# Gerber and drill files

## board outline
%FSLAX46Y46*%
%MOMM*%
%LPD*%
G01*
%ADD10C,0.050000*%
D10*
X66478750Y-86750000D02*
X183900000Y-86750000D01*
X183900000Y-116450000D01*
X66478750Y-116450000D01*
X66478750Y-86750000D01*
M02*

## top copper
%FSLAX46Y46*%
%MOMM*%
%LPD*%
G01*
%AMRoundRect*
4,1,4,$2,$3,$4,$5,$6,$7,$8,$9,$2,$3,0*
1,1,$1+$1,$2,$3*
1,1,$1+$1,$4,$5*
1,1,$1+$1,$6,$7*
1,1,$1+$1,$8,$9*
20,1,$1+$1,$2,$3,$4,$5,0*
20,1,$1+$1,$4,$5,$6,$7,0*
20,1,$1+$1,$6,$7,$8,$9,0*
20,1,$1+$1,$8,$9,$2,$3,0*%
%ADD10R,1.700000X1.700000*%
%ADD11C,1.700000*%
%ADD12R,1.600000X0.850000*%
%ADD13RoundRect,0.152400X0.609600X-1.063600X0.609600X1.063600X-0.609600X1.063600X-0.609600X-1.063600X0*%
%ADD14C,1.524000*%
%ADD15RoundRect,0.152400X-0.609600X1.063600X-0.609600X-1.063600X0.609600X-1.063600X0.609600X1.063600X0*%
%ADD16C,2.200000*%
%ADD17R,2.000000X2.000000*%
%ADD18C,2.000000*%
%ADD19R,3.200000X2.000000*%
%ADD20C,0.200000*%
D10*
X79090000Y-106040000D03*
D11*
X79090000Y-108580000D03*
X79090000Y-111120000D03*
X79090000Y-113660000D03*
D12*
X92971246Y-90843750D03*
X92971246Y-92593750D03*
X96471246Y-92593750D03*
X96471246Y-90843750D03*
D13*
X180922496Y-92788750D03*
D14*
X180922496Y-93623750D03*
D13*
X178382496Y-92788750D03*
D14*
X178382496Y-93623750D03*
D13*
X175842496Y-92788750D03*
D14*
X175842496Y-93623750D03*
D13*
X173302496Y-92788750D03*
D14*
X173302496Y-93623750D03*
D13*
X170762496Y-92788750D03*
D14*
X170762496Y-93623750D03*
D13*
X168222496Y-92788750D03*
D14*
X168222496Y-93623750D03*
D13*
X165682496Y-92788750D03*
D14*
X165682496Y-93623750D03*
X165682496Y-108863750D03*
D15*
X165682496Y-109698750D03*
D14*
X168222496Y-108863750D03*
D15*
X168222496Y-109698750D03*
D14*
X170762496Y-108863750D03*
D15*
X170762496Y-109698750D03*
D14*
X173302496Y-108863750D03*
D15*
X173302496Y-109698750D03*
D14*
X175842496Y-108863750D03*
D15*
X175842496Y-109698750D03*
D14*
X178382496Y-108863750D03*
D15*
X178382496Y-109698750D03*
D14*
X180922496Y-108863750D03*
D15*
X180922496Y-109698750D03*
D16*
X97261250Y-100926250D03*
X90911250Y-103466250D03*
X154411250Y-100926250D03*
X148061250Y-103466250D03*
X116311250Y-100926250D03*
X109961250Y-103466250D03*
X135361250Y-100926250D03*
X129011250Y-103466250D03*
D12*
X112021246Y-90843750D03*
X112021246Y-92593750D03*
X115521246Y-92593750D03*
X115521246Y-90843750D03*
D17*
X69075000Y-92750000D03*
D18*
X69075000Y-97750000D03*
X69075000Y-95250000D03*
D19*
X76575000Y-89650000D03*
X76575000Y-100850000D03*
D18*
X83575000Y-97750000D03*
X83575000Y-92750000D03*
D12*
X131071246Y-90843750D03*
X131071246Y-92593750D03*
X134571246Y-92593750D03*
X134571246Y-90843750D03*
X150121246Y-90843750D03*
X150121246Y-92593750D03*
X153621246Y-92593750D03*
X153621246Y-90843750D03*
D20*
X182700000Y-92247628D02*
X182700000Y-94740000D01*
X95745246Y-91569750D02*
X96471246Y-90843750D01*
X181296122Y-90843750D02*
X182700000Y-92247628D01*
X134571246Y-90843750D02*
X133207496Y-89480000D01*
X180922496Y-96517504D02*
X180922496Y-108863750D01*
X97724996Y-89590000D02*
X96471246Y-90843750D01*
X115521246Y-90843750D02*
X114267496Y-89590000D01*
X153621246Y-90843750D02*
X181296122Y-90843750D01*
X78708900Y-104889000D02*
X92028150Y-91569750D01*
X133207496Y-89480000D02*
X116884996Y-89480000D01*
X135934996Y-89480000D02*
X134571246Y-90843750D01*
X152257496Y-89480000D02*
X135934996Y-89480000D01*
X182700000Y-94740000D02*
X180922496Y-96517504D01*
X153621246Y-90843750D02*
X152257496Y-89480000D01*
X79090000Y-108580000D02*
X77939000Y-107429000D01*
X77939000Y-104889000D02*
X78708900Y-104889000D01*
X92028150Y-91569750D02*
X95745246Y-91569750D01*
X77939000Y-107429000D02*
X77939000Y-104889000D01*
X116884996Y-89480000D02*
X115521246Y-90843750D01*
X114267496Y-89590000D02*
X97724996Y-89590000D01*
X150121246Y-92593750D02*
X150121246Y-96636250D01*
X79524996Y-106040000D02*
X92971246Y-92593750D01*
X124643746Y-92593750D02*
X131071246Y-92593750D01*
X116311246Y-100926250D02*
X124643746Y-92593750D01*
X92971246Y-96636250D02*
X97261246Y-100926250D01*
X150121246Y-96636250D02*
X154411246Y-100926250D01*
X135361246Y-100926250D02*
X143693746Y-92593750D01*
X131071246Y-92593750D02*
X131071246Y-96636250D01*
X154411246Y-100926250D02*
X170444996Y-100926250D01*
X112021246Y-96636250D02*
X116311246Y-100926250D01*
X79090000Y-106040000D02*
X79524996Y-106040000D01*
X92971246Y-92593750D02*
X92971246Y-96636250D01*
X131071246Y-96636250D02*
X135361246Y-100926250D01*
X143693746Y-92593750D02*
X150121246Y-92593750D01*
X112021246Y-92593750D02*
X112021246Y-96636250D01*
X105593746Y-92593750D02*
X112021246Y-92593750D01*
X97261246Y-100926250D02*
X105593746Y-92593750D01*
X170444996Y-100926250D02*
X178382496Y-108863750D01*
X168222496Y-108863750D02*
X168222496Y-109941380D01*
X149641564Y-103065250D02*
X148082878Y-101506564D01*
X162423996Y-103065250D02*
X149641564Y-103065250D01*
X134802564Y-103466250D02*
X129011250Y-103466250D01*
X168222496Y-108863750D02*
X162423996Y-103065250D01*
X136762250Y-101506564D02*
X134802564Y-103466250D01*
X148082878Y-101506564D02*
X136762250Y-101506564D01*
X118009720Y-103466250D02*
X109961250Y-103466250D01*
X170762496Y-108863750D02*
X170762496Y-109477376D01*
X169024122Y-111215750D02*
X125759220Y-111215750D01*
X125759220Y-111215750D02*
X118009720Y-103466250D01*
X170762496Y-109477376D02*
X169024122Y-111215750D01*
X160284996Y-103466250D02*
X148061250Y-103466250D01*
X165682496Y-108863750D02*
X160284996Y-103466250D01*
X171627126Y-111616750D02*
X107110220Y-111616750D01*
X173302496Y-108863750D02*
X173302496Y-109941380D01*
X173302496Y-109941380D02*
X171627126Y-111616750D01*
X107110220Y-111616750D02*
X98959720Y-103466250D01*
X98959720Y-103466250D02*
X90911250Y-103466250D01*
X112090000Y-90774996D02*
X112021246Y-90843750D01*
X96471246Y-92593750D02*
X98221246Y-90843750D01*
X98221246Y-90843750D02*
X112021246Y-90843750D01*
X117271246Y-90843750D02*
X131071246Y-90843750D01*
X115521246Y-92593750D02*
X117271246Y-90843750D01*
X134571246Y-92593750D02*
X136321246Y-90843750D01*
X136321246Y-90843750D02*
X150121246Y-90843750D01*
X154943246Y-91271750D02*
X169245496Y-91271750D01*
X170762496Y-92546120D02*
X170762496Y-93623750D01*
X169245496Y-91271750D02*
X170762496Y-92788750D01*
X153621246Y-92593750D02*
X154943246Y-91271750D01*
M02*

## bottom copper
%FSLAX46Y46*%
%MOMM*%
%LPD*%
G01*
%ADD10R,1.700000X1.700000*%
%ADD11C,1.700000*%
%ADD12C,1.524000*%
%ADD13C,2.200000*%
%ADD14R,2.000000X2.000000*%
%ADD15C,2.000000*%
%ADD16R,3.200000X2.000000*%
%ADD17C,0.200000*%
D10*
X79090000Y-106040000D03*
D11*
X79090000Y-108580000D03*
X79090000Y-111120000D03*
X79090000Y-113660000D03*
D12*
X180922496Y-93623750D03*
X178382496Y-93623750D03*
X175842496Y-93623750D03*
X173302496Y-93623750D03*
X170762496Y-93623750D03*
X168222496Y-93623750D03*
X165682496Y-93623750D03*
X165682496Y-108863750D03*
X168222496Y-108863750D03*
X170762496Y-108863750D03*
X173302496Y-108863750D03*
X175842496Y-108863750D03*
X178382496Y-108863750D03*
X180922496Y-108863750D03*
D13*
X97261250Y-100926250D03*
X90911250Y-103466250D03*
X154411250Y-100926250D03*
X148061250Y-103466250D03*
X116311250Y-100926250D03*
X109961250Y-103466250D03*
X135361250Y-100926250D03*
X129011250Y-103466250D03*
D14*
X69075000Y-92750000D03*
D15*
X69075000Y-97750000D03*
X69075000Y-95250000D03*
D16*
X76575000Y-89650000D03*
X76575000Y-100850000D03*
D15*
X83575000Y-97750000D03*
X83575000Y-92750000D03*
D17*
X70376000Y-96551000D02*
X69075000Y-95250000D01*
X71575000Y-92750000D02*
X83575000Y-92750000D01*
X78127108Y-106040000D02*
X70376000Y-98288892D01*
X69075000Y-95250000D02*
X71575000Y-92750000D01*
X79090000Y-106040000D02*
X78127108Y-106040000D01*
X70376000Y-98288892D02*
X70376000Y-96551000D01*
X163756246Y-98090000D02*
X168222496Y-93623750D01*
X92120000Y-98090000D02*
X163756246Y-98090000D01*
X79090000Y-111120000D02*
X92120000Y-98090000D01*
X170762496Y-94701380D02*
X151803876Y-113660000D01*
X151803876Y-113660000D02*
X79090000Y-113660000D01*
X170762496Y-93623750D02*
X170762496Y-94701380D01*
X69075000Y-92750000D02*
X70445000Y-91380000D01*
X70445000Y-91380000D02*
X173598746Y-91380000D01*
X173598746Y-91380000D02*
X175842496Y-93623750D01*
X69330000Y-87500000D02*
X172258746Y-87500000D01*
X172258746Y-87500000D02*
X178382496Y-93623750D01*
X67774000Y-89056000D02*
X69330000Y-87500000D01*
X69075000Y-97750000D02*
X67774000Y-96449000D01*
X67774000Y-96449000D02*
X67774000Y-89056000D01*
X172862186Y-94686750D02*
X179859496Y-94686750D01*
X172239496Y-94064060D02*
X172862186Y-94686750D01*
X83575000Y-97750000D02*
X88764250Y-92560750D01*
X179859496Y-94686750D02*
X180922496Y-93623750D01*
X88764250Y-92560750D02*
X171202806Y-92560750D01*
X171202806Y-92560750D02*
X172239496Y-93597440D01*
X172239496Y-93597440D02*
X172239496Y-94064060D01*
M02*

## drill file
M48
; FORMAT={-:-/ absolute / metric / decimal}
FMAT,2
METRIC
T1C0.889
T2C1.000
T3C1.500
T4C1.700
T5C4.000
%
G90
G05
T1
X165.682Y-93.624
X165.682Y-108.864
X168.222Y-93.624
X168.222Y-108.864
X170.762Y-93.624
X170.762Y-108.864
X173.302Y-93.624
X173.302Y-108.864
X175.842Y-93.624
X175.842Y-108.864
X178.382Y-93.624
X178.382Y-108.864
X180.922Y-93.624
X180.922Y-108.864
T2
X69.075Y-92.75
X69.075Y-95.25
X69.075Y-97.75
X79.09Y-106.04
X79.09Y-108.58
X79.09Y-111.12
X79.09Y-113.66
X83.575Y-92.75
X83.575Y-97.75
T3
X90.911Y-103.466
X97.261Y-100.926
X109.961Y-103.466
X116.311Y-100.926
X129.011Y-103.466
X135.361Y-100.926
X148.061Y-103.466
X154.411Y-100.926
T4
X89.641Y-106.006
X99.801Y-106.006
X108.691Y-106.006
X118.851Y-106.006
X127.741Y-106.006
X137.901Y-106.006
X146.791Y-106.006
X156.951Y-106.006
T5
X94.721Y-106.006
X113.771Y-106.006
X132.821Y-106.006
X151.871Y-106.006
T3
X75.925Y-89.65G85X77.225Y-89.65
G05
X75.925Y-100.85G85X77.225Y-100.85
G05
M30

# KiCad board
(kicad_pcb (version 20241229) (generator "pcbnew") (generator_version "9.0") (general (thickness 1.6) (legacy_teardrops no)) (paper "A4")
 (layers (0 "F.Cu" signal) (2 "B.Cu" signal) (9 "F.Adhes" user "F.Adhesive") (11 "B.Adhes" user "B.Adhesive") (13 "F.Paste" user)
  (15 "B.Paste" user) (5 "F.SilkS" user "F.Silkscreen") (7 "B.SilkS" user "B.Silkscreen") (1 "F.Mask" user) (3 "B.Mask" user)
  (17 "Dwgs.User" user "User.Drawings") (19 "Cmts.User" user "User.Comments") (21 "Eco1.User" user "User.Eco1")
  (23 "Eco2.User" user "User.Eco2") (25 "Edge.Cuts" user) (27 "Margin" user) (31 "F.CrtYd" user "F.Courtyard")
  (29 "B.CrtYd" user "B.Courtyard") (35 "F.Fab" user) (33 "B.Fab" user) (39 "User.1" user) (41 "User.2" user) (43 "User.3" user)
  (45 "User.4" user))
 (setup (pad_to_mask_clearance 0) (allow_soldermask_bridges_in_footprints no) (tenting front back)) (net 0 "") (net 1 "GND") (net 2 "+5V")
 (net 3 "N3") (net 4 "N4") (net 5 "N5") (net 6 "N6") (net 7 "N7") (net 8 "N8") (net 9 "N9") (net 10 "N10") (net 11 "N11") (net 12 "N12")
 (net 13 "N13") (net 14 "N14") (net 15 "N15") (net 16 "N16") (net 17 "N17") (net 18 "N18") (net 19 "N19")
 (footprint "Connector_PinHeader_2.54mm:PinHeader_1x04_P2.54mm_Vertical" (layer "F.Cu") (at 79.09 106.04)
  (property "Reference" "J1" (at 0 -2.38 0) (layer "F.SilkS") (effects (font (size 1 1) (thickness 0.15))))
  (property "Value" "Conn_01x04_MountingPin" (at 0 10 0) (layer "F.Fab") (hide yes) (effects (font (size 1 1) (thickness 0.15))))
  (pad "1" thru_hole rect (at 0 0) (size 1.7 1.7) (drill 1) (layers "*.Cu" "*.Mask") (remove_unused_layers no) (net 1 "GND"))
  (pad "2" thru_hole circle (at 0 2.54) (size 1.7 1.7) (drill 1) (layers "*.Cu" "*.Mask") (remove_unused_layers no) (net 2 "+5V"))
  (pad "3" thru_hole circle (at 0 5.08) (size 1.7 1.7) (drill 1) (layers "*.Cu" "*.Mask") (remove_unused_layers no) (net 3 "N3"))
  (pad "4" thru_hole circle (at 0 7.62) (size 1.7 1.7) (drill 1) (layers "*.Cu" "*.Mask") (remove_unused_layers no) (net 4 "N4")))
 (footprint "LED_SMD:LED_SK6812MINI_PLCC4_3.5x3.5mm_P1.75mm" (layer "F.Cu") (at 94.721246 91.71875)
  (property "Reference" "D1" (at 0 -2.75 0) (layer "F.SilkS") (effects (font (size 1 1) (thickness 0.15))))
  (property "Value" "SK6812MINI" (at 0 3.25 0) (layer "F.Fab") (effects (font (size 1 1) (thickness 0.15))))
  (pad "1" smd rect (at -1.75 -0.875) (size 1.6 0.85) (layers "F.Cu" "F.Mask" "F.Paste") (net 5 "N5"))
  (pad "2" smd rect (at -1.75 0.875) (size 1.6 0.85) (layers "F.Cu" "F.Mask" "F.Paste") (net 1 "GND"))
  (pad "3" smd rect (at 1.75 0.875) (size 1.6 0.85) (layers "F.Cu" "F.Mask" "F.Paste") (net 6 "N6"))
  (pad "4" smd rect (at 1.75 -0.875) (size 1.6 0.85) (layers "F.Cu" "F.Mask" "F.Paste") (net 2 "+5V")))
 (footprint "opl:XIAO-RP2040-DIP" (layer "F.Cu") (at 173.302496 101.24375 -90)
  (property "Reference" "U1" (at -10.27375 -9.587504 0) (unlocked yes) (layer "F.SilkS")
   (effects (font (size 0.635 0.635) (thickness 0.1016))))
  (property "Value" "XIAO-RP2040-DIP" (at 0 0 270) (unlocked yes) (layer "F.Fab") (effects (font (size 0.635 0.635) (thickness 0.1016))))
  (pad "1" smd roundrect (at -8.455 -7.62 90) (size 2.432 1.524) (layers "F.Cu" "F.Mask") (roundrect_rratio 0.1) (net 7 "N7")
   (thermal_bridge_angle 45))
  (pad "1" thru_hole circle (at -7.62 -7.62 90) (size 1.524 1.524) (drill 0.889) (layers "*.Cu" "*.Mask") (remove_unused_layers no)
   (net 7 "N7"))
  (pad "2" smd roundrect (at -8.455 -5.08 90) (size 2.432 1.524) (layers "F.Cu" "F.Mask") (roundrect_rratio 0.1) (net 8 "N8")
   (thermal_bridge_angle 45))
  (pad "2" thru_hole circle (at -7.62 -5.08 90) (size 1.524 1.524) (drill 0.889) (layers "*.Cu" "*.Mask") (remove_unused_layers no)
   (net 8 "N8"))
  (pad "3" smd roundrect (at -8.455 -2.54 90) (size 2.432 1.524) (layers "F.Cu" "F.Mask") (roundrect_rratio 0.1) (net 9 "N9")
   (thermal_bridge_angle 45))
  (pad "3" thru_hole circle (at -7.62 -2.54 90) (size 1.524 1.524) (drill 0.889) (layers "*.Cu" "*.Mask") (remove_unused_layers no)
   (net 9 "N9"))
  (pad "4" smd roundrect (at -8.455 0 90) (size 2.432 1.524) (layers "F.Cu" "F.Mask") (roundrect_rratio 0.1) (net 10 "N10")
   (thermal_bridge_angle 45))
  (pad "4" thru_hole circle (at -7.62 0 90) (size 1.524 1.524) (drill 0.889) (layers "*.Cu" "*.Mask") (remove_unused_layers no)
   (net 10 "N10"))
  (pad "5" smd roundrect (at -8.455 2.54 90) (size 2.432 1.524) (layers "F.Cu" "F.Mask") (roundrect_rratio 0.1) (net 4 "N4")
   (thermal_bridge_angle 45))
  (pad "5" thru_hole circle (at -7.62 2.54 90) (size 1.524 1.524) (drill 0.889) (layers "*.Cu" "*.Mask") (remove_unused_layers no)
   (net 4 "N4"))
  (pad "6" smd roundrect (at -8.455 5.08 90) (size 2.432 1.524) (layers "F.Cu" "F.Mask") (roundrect_rratio 0.1) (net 3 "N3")
   (thermal_bridge_angle 45))
  (pad "6" thru_hole circle (at -7.62 5.08 90) (size 1.524 1.524) (drill 0.889) (layers "*.Cu" "*.Mask") (remove_unused_layers no)
   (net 3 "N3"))
  (pad "7" smd roundrect (at -8.455 7.62 90) (size 2.432 1.524) (layers "F.Cu" "F.Mask") (roundrect_rratio 0.1) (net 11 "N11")
   (thermal_bridge_angle 45))
  (pad "7" thru_hole circle (at -7.62 7.62 90) (size 1.524 1.524) (drill 0.889) (layers "*.Cu" "*.Mask") (remove_unused_layers no)
   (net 11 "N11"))
  (pad "8" thru_hole circle (at 7.62 7.62 270) (size 1.524 1.524) (drill 0.889) (layers "*.Cu" "*.Mask") (remove_unused_layers no)
   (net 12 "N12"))
  (pad "8" smd roundrect (at 8.455 7.62 270) (size 2.432 1.524) (layers "F.Cu" "F.Mask") (roundrect_rratio 0.1) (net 12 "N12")
   (thermal_bridge_angle 45))
  (pad "9" thru_hole circle (at 7.62 5.08 270) (size 1.524 1.524) (drill 0.889) (layers "*.Cu" "*.Mask") (remove_unused_layers no)
   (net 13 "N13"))
  (pad "9" smd roundrect (at 8.455 5.08 270) (size 2.432 1.524) (layers "F.Cu" "F.Mask") (roundrect_rratio 0.1) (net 13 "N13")
   (thermal_bridge_angle 45))
  (pad "10" thru_hole circle (at 7.62 2.54 270) (size 1.524 1.524) (drill 0.889) (layers "*.Cu" "*.Mask") (remove_unused_layers no)
   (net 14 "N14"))
  (pad "10" smd roundrect (at 8.455 2.54 270) (size 2.432 1.524) (layers "F.Cu" "F.Mask") (roundrect_rratio 0.1) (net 14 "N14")
   (thermal_bridge_angle 45))
  (pad "11" thru_hole circle (at 7.62 0 270) (size 1.524 1.524) (drill 0.889) (layers "*.Cu" "*.Mask") (remove_unused_layers no)
   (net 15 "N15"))
  (pad "11" smd roundrect (at 8.455 0 270) (size 2.432 1.524) (layers "F.Cu" "F.Mask") (roundrect_rratio 0.1) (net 15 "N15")
   (thermal_bridge_angle 45))
  (pad "12" thru_hole circle (at 7.62 -2.54 270) (size 1.524 1.524) (drill 0.889) (layers "*.Cu" "*.Mask") (remove_unused_layers no)
   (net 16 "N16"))
  (pad "12" smd roundrect (at 8.455 -2.54 270) (size 2.432 1.524) (layers "F.Cu" "F.Mask") (roundrect_rratio 0.1) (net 16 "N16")
   (thermal_bridge_angle 45))
  (pad "13" thru_hole circle (at 7.62 -5.08 270) (size 1.524 1.524) (drill 0.889) (layers "*.Cu" "*.Mask") (remove_unused_layers no)
   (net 1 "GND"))
  (pad "13" smd roundrect (at 8.455 -5.08 270) (size 2.432 1.524) (layers "F.Cu" "F.Mask") (roundrect_rratio 0.1) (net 1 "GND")
   (thermal_bridge_angle 45))
  (pad "14" thru_hole circle (at 7.62 -7.62 270) (size 1.524 1.524) (drill 0.889) (layers "*.Cu" "*.Mask") (remove_unused_layers no)
   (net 2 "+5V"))
  (pad "14" smd roundrect (at 8.455 -7.62 270) (size 2.432 1.524) (layers "F.Cu" "F.Mask") (roundrect_rratio 0.1) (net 2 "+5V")
   (thermal_bridge_angle 45)))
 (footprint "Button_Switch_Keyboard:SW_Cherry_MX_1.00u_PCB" (layer "F.Cu") (at 97.26125 100.92625)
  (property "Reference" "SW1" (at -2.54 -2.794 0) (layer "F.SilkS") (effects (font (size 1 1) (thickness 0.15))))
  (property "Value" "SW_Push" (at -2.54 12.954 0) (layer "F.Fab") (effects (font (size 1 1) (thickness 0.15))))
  (pad "" np_thru_hole circle (at -7.62 5.08) (size 1.7 1.7) (drill 1.7) (layers "*.Cu" "*.Mask"))
  (pad "" np_thru_hole circle (at -2.54 5.08) (size 4 4) (drill 4) (layers "*.Cu" "*.Mask"))
  (pad "" np_thru_hole circle (at 2.54 5.08) (size 1.7 1.7) (drill 1.7) (layers "*.Cu" "*.Mask"))
  (pad "1" thru_hole circle (at 0 0) (size 2.2 2.2) (drill 1.5) (layers "*.Cu" "*.Mask") (remove_unused_layers no) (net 1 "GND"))
  (pad "2" thru_hole circle (at -6.35 2.54) (size 2.2 2.2) (drill 1.5) (layers "*.Cu" "*.Mask") (remove_unused_layers no) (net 15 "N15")))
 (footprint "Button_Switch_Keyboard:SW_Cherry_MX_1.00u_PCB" (layer "F.Cu") (at 154.41125 100.92625)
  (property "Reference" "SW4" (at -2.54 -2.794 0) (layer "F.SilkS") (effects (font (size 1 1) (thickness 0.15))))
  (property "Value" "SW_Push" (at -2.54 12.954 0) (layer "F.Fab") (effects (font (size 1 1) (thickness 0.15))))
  (pad "" np_thru_hole circle (at -7.62 5.08) (size 1.7 1.7) (drill 1.7) (layers "*.Cu" "*.Mask"))
  (pad "" np_thru_hole circle (at -2.54 5.08) (size 4 4) (drill 4) (layers "*.Cu" "*.Mask"))
  (pad "" np_thru_hole circle (at 2.54 5.08) (size 1.7 1.7) (drill 1.7) (layers "*.Cu" "*.Mask"))
  (pad "1" thru_hole circle (at 0 0) (size 2.2 2.2) (drill 1.5) (layers "*.Cu" "*.Mask") (remove_unused_layers no) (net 1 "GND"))
  (pad "2" thru_hole circle (at -6.35 2.54) (size 2.2 2.2) (drill 1.5) (layers "*.Cu" "*.Mask") (remove_unused_layers no) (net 12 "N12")))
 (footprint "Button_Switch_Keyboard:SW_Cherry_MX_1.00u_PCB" (layer "F.Cu") (at 116.31125 100.92625)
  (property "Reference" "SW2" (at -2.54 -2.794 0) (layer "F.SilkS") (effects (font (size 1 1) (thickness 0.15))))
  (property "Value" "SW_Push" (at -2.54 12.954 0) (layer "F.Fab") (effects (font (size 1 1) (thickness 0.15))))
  (pad "" np_thru_hole circle (at -7.62 5.08) (size 1.7 1.7) (drill 1.7) (layers "*.Cu" "*.Mask"))
  (pad "" np_thru_hole circle (at -2.54 5.08) (size 4 4) (drill 4) (layers "*.Cu" "*.Mask"))
  (pad "" np_thru_hole circle (at 2.54 5.08) (size 1.7 1.7) (drill 1.7) (layers "*.Cu" "*.Mask"))
  (pad "1" thru_hole circle (at 0 0) (size 2.2 2.2) (drill 1.5) (layers "*.Cu" "*.Mask") (remove_unused_layers no) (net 1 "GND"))
  (pad "2" thru_hole circle (at -6.35 2.54) (size 2.2 2.2) (drill 1.5) (layers "*.Cu" "*.Mask") (remove_unused_layers no) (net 14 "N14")))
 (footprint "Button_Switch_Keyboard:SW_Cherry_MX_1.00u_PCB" (layer "F.Cu") (at 135.36125 100.92625)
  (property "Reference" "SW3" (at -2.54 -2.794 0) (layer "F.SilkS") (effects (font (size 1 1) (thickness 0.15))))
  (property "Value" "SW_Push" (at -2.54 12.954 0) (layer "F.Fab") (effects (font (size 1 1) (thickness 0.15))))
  (pad "" np_thru_hole circle (at -7.62 5.08) (size 1.7 1.7) (drill 1.7) (layers "*.Cu" "*.Mask"))
  (pad "" np_thru_hole circle (at -2.54 5.08) (size 4 4) (drill 4) (layers "*.Cu" "*.Mask"))
  (pad "" np_thru_hole circle (at 2.54 5.08) (size 1.7 1.7) (drill 1.7) (layers "*.Cu" "*.Mask"))
  (pad "1" thru_hole circle (at 0 0) (size 2.2 2.2) (drill 1.5) (layers "*.Cu" "*.Mask") (remove_unused_layers no) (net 1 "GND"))
  (pad "2" thru_hole circle (at -6.35 2.54) (size 2.2 2.2) (drill 1.5) (layers "*.Cu" "*.Mask") (remove_unused_layers no) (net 13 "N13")))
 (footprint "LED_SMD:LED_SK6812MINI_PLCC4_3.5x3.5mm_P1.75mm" (layer "F.Cu") (at 113.771246 91.71875)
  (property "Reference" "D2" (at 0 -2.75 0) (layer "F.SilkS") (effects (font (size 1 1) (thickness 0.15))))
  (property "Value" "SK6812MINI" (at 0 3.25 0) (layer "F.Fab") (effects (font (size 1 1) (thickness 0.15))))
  (pad "1" smd rect (at -1.75 -0.875) (size 1.6 0.85) (layers "F.Cu" "F.Mask" "F.Paste") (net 6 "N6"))
  (pad "2" smd rect (at -1.75 0.875) (size 1.6 0.85) (layers "F.Cu" "F.Mask" "F.Paste") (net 1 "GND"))
  (pad "3" smd rect (at 1.75 0.875) (size 1.6 0.85) (layers "F.Cu" "F.Mask" "F.Paste") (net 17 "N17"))
  (pad "4" smd rect (at 1.75 -0.875) (size 1.6 0.85) (layers "F.Cu" "F.Mask" "F.Paste") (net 2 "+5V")))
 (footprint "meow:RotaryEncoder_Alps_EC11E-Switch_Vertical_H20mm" (layer "F.Cu") (at 69.075 92.75)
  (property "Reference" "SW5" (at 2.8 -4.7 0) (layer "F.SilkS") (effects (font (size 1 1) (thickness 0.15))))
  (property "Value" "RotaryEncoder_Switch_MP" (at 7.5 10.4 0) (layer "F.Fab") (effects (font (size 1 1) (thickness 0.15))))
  (pad "A" thru_hole rect (at 0 0) (size 2 2) (drill 1) (layers "*.Cu" "*.Mask") (remove_unused_layers no) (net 9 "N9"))
  (pad "B" thru_hole circle (at 0 5) (size 2 2) (drill 1) (layers "*.Cu" "*.Mask") (remove_unused_layers no) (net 8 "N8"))
  (pad "C" thru_hole circle (at 0 2.5) (size 2 2) (drill 1) (layers "*.Cu" "*.Mask") (remove_unused_layers no) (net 1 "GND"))
  (pad "MP" thru_hole rect (at 7.5 -3.1) (size 3.2 2) (drill oval 2.8 1.5) (layers "*.Cu" "*.Mask") (remove_unused_layers no) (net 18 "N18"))
  (pad "MP" thru_hole rect (at 7.5 8.1) (size 3.2 2) (drill oval 2.8 1.5) (layers "*.Cu" "*.Mask") (remove_unused_layers no) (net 18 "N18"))
  (pad "S1" thru_hole circle (at 14.5 5) (size 2 2) (drill 1) (layers "*.Cu" "*.Mask") (remove_unused_layers no) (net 7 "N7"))
  (pad "S2" thru_hole circle (at 14.5 0) (size 2 2) (drill 1) (layers "*.Cu" "*.Mask") (remove_unused_layers no) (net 1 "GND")))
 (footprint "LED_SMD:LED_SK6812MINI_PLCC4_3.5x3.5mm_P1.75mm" (layer "F.Cu") (at 132.821246 91.71875)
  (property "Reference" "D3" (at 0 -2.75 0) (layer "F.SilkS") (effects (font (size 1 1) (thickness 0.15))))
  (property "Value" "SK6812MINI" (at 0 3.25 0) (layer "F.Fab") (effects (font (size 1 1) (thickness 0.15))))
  (pad "1" smd rect (at -1.75 -0.875) (size 1.6 0.85) (layers "F.Cu" "F.Mask" "F.Paste") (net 17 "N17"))
  (pad "2" smd rect (at -1.75 0.875) (size 1.6 0.85) (layers "F.Cu" "F.Mask" "F.Paste") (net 1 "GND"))
  (pad "3" smd rect (at 1.75 0.875) (size 1.6 0.85) (layers "F.Cu" "F.Mask" "F.Paste") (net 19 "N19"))
  (pad "4" smd rect (at 1.75 -0.875) (size 1.6 0.85) (layers "F.Cu" "F.Mask" "F.Paste") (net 2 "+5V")))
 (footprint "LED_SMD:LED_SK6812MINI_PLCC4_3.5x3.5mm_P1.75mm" (layer "F.Cu") (at 151.871246 91.71875)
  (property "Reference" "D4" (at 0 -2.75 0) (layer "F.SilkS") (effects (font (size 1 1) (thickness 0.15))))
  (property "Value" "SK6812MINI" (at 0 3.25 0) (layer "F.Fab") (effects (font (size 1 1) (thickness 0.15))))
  (pad "1" smd rect (at -1.75 -0.875) (size 1.6 0.85) (layers "F.Cu" "F.Mask" "F.Paste") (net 19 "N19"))
  (pad "2" smd rect (at -1.75 0.875) (size 1.6 0.85) (layers "F.Cu" "F.Mask" "F.Paste") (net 1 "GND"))
  (pad "3" smd rect (at 1.75 0.875) (size 1.6 0.85) (layers "F.Cu" "F.Mask" "F.Paste") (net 4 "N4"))
  (pad "4" smd rect (at 1.75 -0.875) (size 1.6 0.85) (layers "F.Cu" "F.Mask" "F.Paste") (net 2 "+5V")))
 (gr_rect (start 66.47875 86.75) (end 183.9 116.45) (stroke (width 0.05) (type default)) (fill no) (layer "Edge.Cuts"))
 (segment (start 182.7 92.247628) (end 182.7 94.74) (width 0.2) (layer "F.Cu") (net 2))
 (segment (start 95.745246 91.56975) (end 96.471246 90.84375) (width 0.2) (layer "F.Cu") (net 2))
 (segment (start 181.296122 90.84375) (end 182.7 92.247628) (width 0.2) (layer "F.Cu") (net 2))
 (segment (start 134.571246 90.84375) (end 133.207496 89.48) (width 0.2) (layer "F.Cu") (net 2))
 (segment (start 180.922496 96.517504) (end 180.922496 108.86375) (width 0.2) (layer "F.Cu") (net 2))
 (segment (start 97.724996 89.59) (end 96.471246 90.84375) (width 0.2) (layer "F.Cu") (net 2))
 (segment (start 115.521246 90.84375) (end 114.267496 89.59) (width 0.2) (layer "F.Cu") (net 2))
 (segment (start 153.621246 90.84375) (end 181.296122 90.84375) (width 0.2) (layer "F.Cu") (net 2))
 (segment (start 78.7089 104.889) (end 92.02815 91.56975) (width 0.2) (layer "F.Cu") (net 2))
 (segment (start 133.207496 89.48) (end 116.884996 89.48) (width 0.2) (layer "F.Cu") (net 2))
 (segment (start 135.934996 89.48) (end 134.571246 90.84375) (width 0.2) (layer "F.Cu") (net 2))
 (segment (start 152.257496 89.48) (end 135.934996 89.48) (width 0.2) (layer "F.Cu") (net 2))
 (segment (start 182.7 94.74) (end 180.922496 96.517504) (width 0.2) (layer "F.Cu") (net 2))
 (segment (start 153.621246 90.84375) (end 152.257496 89.48) (width 0.2) (layer "F.Cu") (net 2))
 (segment (start 79.09 108.58) (end 77.939 107.429) (width 0.2) (layer "F.Cu") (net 2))
 (segment (start 77.939 104.889) (end 78.7089 104.889) (width 0.2) (layer "F.Cu") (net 2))
 (segment (start 92.02815 91.56975) (end 95.745246 91.56975) (width 0.2) (layer "F.Cu") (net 2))
 (segment (start 77.939 107.429) (end 77.939 104.889) (width 0.2) (layer "F.Cu") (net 2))
 (segment (start 116.884996 89.48) (end 115.521246 90.84375) (width 0.2) (layer "F.Cu") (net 2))
 (segment (start 114.267496 89.59) (end 97.724996 89.59) (width 0.2) (layer "F.Cu") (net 2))
 (segment (start 150.121246 92.59375) (end 150.121246 96.63625) (width 0.2) (layer "F.Cu") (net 1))
 (segment (start 79.524996 106.04) (end 92.971246 92.59375) (width 0.2) (layer "F.Cu") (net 1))
 (segment (start 124.643746 92.59375) (end 131.071246 92.59375) (width 0.2) (layer "F.Cu") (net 1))
 (segment (start 116.311246 100.92625) (end 124.643746 92.59375) (width 0.2) (layer "F.Cu") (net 1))
 (segment (start 92.971246 96.63625) (end 97.261246 100.92625) (width 0.2) (layer "F.Cu") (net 1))
 (segment (start 150.121246 96.63625) (end 154.411246 100.92625) (width 0.2) (layer "F.Cu") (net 1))
 (segment (start 135.361246 100.92625) (end 143.693746 92.59375) (width 0.2) (layer "F.Cu") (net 1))
 (segment (start 131.071246 92.59375) (end 131.071246 96.63625) (width 0.2) (layer "F.Cu") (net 1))
 (segment (start 154.411246 100.92625) (end 170.444996 100.92625) (width 0.2) (layer "F.Cu") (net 1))
 (segment (start 112.021246 96.63625) (end 116.311246 100.92625) (width 0.2) (layer "F.Cu") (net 1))
 (segment (start 79.09 106.04) (end 79.524996 106.04) (width 0.2) (layer "F.Cu") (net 1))
 (segment (start 92.971246 92.59375) (end 92.971246 96.63625) (width 0.2) (layer "F.Cu") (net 1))
 (segment (start 131.071246 96.63625) (end 135.361246 100.92625) (width 0.2) (layer "F.Cu") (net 1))
 (segment (start 143.693746 92.59375) (end 150.121246 92.59375) (width 0.2) (layer "F.Cu") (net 1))
 (segment (start 112.021246 92.59375) (end 112.021246 96.63625) (width 0.2) (layer "F.Cu") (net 1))
 (segment (start 105.593746 92.59375) (end 112.021246 92.59375) (width 0.2) (layer "F.Cu") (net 1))
 (segment (start 97.261246 100.92625) (end 105.593746 92.59375) (width 0.2) (layer "F.Cu") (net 1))
 (segment (start 170.444996 100.92625) (end 178.382496 108.86375) (width 0.2) (layer "F.Cu") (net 1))
 (segment (start 70.376 96.551) (end 69.075 95.25) (width 0.2) (layer "B.Cu") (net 1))
 (segment (start 71.575 92.75) (end 83.575 92.75) (width 0.2) (layer "B.Cu") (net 1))
 (segment (start 78.127108 106.04) (end 70.376 98.288892) (width 0.2) (layer "B.Cu") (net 1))
 (segment (start 69.075 95.25) (end 71.575 92.75) (width 0.2) (layer "B.Cu") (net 1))
 (segment (start 79.09 106.04) (end 78.127108 106.04) (width 0.2) (layer "B.Cu") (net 1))
 (segment (start 70.376 98.288892) (end 70.376 96.551) (width 0.2) (layer "B.Cu") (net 1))
 (segment (start 168.222496 108.86375) (end 168.222496 109.94138) (width 0.2) (layer "F.Cu") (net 13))
 (segment (start 149.641564 103.06525) (end 148.082878 101.506564) (width 0.2) (layer "F.Cu") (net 13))
 (segment (start 162.423996 103.06525) (end 149.641564 103.06525) (width 0.2) (layer "F.Cu") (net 13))
 (segment (start 134.802564 103.46625) (end 129.01125 103.46625) (width 0.2) (layer "F.Cu") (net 13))
 (segment (start 168.222496 108.86375) (end 162.423996 103.06525) (width 0.2) (layer "F.Cu") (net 13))
 (segment (start 136.76225 101.506564) (end 134.802564 103.46625) (width 0.2) (layer "F.Cu") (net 13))
 (segment (start 148.082878 101.506564) (end 136.76225 101.506564) (width 0.2) (layer "F.Cu") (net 13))
 (segment (start 118.00972 103.46625) (end 109.96125 103.46625) (width 0.2) (layer "F.Cu") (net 14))
 (segment (start 170.762496 108.86375) (end 170.762496 109.477376) (width 0.2) (layer "F.Cu") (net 14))
 (segment (start 169.024122 111.21575) (end 125.75922 111.21575) (width 0.2) (layer "F.Cu") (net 14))
 (segment (start 125.75922 111.21575) (end 118.00972 103.46625) (width 0.2) (layer "F.Cu") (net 14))
 (segment (start 170.762496 109.477376) (end 169.024122 111.21575) (width 0.2) (layer "F.Cu") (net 14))
 (segment (start 160.284996 103.46625) (end 148.06125 103.46625) (width 0.2) (layer "F.Cu") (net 12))
 (segment (start 165.682496 108.86375) (end 160.284996 103.46625) (width 0.2) (layer "F.Cu") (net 12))
 (segment (start 163.756246 98.09) (end 168.222496 93.62375) (width 0.2) (layer "B.Cu") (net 3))
 (segment (start 92.12 98.09) (end 163.756246 98.09) (width 0.2) (layer "B.Cu") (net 3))
 (segment (start 79.09 111.12) (end 92.12 98.09) (width 0.2) (layer "B.Cu") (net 3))
 (segment (start 171.627126 111.61675) (end 107.11022 111.61675) (width 0.2) (layer "F.Cu") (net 15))
 (segment (start 173.302496 108.86375) (end 173.302496 109.94138) (width 0.2) (layer "F.Cu") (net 15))
 (segment (start 173.302496 109.94138) (end 171.627126 111.61675) (width 0.2) (layer "F.Cu") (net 15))
 (segment (start 107.11022 111.61675) (end 98.95972 103.46625) (width 0.2) (layer "F.Cu") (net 15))
 (segment (start 98.95972 103.46625) (end 90.91125 103.46625) (width 0.2) (layer "F.Cu") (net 15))
 (segment (start 112.09 90.774996) (end 112.021246 90.84375) (width 0.2) (layer "F.Cu") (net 6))
 (segment (start 96.471246 92.59375) (end 98.221246 90.84375) (width 0.2) (layer "F.Cu") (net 6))
 (segment (start 98.221246 90.84375) (end 112.021246 90.84375) (width 0.2) (layer "F.Cu") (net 6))
 (segment (start 117.271246 90.84375) (end 131.071246 90.84375) (width 0.2) (layer "F.Cu") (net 17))
 (segment (start 115.521246 92.59375) (end 117.271246 90.84375) (width 0.2) (layer "F.Cu") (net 17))
 (segment (start 134.571246 92.59375) (end 136.321246 90.84375) (width 0.2) (layer "F.Cu") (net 19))
 (segment (start 136.321246 90.84375) (end 150.121246 90.84375) (width 0.2) (layer "F.Cu") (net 19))
 (segment (start 154.943246 91.27175) (end 169.245496 91.27175) (width 0.2) (layer "F.Cu") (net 4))
 (segment (start 170.762496 92.54612) (end 170.762496 93.62375) (width 0.2) (layer "F.Cu") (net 4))
 (segment (start 169.245496 91.27175) (end 170.762496 92.78875) (width 0.2) (layer "F.Cu") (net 4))
 (segment (start 153.621246 92.59375) (end 154.943246 91.27175) (width 0.2) (layer "F.Cu") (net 4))
 (segment (start 170.762496 94.70138) (end 151.803876 113.66) (width 0.2) (layer "B.Cu") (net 4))
 (segment (start 151.803876 113.66) (end 79.09 113.66) (width 0.2) (layer "B.Cu") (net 4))
 (segment (start 170.762496 93.62375) (end 170.762496 94.70138) (width 0.2) (layer "B.Cu") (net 4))
 (segment (start 69.075 92.75) (end 70.445 91.38) (width 0.2) (layer "B.Cu") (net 9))
 (segment (start 70.445 91.38) (end 173.598746 91.38) (width 0.2) (layer "B.Cu") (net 9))
 (segment (start 173.598746 91.38) (end 175.842496 93.62375) (width 0.2) (layer "B.Cu") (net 9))
 (segment (start 69.33 87.5) (end 172.258746 87.5) (width 0.2) (layer "B.Cu") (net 8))
 (segment (start 172.258746 87.5) (end 178.382496 93.62375) (width 0.2) (layer "B.Cu") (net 8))
 (segment (start 67.774 89.056) (end 69.33 87.5) (width 0.2) (layer "B.Cu") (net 8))
 (segment (start 69.075 97.75) (end 67.774 96.449) (width 0.2) (layer "B.Cu") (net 8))
 (segment (start 67.774 96.449) (end 67.774 89.056) (width 0.2) (layer "B.Cu") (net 8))
 (segment (start 172.862186 94.68675) (end 179.859496 94.68675) (width 0.2) (layer "B.Cu") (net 7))
 (segment (start 172.239496 94.06406) (end 172.862186 94.68675) (width 0.2) (layer "B.Cu") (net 7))
 (segment (start 83.575 97.75) (end 88.76425 92.56075) (width 0.2) (layer "B.Cu") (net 7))
 (segment (start 179.859496 94.68675) (end 180.922496 93.62375) (width 0.2) (layer "B.Cu") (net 7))
 (segment (start 88.76425 92.56075) (end 171.202806 92.56075) (width 0.2) (layer "B.Cu") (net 7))
 (segment (start 171.202806 92.56075) (end 172.239496 93.59744) (width 0.2) (layer "B.Cu") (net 7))
 (segment (start 172.239496 93.59744) (end 172.239496 94.06406) (width 0.2) (layer "B.Cu") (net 7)))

